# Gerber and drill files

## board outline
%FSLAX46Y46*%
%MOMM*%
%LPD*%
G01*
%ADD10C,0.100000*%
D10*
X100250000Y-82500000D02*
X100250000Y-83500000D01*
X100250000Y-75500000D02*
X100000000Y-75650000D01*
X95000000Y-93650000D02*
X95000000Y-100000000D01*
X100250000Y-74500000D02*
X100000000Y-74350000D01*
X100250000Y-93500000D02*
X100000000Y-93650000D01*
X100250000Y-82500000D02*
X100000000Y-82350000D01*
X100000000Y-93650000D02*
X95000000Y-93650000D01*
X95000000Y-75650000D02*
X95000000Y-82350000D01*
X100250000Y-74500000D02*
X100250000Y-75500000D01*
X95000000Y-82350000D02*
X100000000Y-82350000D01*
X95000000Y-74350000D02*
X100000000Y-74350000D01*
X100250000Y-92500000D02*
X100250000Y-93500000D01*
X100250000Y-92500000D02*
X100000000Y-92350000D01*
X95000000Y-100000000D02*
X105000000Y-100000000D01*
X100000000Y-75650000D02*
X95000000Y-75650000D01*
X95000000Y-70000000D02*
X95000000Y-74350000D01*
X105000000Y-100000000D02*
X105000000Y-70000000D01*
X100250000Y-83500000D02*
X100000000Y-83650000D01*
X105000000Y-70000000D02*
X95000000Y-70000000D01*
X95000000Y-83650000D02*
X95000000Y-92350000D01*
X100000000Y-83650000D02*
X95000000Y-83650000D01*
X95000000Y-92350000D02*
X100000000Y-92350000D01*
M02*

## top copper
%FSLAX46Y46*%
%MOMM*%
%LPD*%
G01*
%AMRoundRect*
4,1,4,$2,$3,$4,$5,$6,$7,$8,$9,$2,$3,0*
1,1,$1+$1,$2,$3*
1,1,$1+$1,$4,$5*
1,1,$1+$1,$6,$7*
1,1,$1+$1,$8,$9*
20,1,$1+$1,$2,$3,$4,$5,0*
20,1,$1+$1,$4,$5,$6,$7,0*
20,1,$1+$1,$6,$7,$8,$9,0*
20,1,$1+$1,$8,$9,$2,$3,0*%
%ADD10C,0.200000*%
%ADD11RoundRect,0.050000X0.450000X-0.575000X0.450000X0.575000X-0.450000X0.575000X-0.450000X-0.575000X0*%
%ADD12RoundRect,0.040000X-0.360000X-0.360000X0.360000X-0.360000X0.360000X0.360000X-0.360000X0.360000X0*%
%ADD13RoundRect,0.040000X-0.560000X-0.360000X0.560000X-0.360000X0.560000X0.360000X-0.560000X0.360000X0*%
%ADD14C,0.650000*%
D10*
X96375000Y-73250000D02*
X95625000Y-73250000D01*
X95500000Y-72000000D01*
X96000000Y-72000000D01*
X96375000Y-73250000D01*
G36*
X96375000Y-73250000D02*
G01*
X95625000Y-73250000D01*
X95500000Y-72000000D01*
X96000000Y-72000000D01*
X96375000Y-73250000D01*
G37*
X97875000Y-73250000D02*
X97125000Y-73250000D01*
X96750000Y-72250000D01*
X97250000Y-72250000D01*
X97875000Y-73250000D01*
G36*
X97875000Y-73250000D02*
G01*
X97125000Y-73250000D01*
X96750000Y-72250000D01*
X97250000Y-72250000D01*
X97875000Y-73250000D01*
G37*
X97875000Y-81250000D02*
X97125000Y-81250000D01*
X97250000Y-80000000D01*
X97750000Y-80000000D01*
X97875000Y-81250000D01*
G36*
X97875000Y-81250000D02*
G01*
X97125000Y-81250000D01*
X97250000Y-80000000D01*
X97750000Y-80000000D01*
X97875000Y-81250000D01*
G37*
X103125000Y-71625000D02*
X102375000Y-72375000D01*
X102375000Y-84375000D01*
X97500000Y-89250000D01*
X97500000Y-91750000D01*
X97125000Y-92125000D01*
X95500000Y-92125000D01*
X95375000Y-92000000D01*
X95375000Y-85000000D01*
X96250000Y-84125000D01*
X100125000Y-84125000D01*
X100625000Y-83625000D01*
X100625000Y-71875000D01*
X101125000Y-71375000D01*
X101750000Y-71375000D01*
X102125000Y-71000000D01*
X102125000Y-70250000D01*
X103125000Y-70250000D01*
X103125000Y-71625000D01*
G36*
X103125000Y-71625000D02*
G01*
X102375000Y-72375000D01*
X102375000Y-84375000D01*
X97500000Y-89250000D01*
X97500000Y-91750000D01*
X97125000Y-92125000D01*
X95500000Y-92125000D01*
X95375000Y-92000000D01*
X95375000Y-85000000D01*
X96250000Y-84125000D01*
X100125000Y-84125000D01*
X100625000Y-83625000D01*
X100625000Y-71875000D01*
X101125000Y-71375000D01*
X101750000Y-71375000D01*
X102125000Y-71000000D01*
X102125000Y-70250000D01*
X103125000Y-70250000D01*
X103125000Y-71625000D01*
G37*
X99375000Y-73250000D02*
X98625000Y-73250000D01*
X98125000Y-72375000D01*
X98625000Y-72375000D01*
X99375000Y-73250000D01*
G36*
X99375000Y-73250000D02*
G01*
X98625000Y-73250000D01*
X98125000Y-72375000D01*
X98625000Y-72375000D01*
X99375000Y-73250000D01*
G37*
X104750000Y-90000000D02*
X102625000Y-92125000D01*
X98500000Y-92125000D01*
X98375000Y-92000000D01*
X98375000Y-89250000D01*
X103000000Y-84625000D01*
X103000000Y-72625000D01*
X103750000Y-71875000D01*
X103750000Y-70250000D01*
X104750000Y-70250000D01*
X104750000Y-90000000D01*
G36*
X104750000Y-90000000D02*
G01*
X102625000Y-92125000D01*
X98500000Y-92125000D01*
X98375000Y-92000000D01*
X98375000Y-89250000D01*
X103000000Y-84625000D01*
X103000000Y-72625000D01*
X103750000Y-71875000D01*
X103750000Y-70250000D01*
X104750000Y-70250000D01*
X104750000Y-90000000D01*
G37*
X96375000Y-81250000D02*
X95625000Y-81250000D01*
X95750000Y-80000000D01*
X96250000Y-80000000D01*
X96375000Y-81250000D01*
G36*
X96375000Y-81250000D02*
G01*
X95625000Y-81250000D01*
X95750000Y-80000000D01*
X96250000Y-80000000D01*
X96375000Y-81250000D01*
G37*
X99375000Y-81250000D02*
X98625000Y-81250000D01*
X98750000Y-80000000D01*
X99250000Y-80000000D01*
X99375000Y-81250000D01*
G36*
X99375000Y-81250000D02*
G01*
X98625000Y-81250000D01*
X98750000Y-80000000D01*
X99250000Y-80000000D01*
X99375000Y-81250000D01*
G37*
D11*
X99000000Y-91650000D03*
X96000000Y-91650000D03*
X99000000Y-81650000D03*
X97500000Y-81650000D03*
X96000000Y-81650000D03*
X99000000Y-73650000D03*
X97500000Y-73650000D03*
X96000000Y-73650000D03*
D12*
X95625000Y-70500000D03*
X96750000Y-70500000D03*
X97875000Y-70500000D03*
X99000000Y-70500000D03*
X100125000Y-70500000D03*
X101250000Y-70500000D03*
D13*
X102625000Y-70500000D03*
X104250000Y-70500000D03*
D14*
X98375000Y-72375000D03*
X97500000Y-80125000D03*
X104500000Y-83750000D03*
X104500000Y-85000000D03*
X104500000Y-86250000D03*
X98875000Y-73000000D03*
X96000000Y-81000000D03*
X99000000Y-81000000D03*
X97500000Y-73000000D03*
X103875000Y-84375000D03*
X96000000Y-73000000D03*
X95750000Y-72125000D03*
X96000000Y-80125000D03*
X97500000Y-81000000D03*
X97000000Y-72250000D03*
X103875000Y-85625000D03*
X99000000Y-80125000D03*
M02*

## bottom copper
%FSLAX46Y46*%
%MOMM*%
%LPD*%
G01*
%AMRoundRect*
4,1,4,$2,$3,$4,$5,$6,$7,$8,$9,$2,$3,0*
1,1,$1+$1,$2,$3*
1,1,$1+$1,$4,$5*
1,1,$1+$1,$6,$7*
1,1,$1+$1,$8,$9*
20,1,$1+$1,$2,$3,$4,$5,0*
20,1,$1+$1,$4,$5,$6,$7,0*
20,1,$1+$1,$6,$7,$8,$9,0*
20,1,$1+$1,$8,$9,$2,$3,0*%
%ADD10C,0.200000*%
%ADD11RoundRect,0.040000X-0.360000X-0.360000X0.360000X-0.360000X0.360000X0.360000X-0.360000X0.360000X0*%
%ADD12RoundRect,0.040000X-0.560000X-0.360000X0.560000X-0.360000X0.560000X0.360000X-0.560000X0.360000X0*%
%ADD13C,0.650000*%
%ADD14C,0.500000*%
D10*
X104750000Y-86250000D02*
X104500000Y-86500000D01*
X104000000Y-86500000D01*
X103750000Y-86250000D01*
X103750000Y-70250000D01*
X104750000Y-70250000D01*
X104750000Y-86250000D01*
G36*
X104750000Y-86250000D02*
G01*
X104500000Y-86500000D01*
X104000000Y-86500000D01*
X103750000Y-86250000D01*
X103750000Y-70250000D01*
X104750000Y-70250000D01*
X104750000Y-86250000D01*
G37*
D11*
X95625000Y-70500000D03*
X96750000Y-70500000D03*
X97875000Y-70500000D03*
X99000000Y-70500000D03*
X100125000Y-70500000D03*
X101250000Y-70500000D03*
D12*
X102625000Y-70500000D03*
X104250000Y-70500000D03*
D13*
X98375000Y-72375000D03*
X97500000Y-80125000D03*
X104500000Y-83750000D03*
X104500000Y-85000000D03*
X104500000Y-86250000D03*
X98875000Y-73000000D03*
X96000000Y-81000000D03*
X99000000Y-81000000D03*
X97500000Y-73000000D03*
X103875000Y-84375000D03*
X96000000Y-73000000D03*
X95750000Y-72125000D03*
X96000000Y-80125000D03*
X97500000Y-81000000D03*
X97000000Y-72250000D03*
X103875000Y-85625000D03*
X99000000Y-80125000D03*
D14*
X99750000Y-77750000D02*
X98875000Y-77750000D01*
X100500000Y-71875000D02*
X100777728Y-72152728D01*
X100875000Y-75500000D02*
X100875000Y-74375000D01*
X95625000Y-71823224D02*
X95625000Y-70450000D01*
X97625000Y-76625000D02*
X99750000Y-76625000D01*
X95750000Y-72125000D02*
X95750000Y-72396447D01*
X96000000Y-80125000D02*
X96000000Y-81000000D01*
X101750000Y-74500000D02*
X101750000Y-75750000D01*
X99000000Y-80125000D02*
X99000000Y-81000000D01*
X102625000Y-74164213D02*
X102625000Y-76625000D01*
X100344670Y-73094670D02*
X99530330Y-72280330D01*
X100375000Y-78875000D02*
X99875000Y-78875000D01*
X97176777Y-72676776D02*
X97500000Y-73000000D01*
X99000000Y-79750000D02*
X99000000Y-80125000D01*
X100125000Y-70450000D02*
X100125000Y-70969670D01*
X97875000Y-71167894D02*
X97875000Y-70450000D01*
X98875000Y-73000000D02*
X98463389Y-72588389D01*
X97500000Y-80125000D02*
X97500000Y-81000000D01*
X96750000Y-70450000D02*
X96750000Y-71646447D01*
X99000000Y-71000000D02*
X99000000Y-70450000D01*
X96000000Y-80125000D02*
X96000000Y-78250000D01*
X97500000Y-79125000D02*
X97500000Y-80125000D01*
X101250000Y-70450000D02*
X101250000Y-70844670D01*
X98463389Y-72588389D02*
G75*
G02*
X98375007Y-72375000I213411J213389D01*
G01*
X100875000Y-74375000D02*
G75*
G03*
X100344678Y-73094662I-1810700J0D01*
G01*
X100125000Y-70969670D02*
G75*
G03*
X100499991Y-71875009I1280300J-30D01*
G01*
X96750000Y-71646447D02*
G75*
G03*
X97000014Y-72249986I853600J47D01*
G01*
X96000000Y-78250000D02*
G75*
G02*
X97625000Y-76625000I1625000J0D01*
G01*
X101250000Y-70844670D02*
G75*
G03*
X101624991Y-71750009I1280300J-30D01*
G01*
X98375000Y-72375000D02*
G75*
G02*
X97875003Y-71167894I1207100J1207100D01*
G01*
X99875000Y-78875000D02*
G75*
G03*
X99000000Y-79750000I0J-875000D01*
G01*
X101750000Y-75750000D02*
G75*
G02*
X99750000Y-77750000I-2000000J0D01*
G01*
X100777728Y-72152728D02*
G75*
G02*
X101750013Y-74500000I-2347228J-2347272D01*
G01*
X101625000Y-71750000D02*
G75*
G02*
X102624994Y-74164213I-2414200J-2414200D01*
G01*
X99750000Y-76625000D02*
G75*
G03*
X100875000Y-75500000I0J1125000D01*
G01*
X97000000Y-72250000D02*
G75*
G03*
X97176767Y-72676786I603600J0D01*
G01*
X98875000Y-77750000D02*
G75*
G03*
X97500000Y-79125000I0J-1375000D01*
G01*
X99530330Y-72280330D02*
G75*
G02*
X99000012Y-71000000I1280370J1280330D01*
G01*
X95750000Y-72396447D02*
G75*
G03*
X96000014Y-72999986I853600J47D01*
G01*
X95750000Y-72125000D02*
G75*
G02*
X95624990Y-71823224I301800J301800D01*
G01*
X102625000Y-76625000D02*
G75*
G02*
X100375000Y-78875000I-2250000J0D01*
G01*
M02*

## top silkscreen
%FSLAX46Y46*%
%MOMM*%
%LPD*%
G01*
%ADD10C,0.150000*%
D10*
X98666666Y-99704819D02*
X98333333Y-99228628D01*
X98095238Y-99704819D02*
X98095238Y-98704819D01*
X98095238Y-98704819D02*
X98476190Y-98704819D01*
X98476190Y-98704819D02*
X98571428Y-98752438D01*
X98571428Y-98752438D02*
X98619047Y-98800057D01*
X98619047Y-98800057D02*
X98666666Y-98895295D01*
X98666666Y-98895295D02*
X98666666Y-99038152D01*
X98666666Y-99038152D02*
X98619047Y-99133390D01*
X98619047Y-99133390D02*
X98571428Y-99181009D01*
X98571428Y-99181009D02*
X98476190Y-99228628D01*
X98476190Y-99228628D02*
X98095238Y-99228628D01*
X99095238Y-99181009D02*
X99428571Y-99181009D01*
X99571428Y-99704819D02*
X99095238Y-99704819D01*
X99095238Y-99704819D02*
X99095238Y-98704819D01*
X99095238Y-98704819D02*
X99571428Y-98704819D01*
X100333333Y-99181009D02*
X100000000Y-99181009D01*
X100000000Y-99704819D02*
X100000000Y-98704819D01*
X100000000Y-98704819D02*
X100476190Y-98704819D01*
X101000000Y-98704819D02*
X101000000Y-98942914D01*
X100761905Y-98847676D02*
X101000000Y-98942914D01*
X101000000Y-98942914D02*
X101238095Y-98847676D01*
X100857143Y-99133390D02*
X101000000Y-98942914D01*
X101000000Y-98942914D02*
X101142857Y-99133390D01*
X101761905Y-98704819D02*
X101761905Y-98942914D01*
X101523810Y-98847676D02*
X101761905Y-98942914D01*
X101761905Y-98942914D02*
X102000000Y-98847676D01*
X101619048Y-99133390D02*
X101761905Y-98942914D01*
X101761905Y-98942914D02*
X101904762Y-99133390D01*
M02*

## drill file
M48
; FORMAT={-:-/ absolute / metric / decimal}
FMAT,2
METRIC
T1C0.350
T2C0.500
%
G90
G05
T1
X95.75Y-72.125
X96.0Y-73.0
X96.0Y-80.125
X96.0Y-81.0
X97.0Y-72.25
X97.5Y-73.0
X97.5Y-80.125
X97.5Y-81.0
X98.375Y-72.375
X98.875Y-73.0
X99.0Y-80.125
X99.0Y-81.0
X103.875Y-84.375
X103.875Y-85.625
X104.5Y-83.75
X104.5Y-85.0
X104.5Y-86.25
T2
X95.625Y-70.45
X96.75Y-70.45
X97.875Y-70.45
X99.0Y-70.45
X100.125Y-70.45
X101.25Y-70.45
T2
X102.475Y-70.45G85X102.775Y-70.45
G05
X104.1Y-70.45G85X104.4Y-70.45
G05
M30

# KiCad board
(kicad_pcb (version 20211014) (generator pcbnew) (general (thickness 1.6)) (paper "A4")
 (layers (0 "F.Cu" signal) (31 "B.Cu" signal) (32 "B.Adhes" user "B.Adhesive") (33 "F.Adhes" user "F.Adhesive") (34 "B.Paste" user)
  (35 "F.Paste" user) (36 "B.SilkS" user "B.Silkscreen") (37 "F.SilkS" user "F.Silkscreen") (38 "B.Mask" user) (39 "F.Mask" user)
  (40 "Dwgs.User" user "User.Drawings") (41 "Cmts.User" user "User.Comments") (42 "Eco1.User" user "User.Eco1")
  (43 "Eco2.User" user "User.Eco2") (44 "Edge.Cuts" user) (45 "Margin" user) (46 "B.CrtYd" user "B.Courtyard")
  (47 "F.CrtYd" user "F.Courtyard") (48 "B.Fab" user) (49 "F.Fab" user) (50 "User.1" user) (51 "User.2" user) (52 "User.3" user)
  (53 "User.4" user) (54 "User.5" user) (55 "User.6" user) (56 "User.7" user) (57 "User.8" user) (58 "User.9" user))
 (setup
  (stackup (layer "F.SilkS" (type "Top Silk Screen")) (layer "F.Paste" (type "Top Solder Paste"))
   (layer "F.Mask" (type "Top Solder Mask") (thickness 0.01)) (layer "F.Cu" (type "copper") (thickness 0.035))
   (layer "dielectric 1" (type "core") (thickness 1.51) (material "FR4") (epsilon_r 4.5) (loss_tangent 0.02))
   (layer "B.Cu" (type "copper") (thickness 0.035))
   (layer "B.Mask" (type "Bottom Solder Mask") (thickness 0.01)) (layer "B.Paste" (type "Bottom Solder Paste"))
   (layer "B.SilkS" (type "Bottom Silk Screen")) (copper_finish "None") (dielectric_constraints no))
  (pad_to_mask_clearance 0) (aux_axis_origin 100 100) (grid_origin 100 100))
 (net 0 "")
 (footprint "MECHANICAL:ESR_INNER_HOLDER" (layer "F.Cu") (at 100 100)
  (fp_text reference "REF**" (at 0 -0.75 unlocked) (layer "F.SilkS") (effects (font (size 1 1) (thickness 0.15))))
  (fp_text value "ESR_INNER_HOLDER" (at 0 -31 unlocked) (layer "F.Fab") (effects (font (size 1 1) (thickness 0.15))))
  (fp_line (start 0.25 -17.5) (end 0.25 -16.5) (layer "Edge.Cuts") (width 0.1))
  (fp_line (start 0.25 -24.5) (end 0 -24.35) (layer "Edge.Cuts") (width 0.1))
  (fp_line (start -5 -6.35) (end -5 0) (layer "Edge.Cuts") (width 0.1))
  (fp_line (start 0.25 -25.5) (end 0 -25.65) (layer "Edge.Cuts") (width 0.1))
  (fp_line (start 0.25 -6.5) (end 0 -6.35) (layer "Edge.Cuts") (width 0.1))
  (fp_line (start 0.25 -17.5) (end 0 -17.65) (layer "Edge.Cuts") (width 0.1))
  (fp_line (start 0 -6.35) (end -5 -6.35) (layer "Edge.Cuts") (width 0.1))
  (fp_line (start -5 -24.35) (end -5 -17.65) (layer "Edge.Cuts") (width 0.1))
  (fp_line (start 0.25 -25.5) (end 0.25 -24.5) (layer "Edge.Cuts") (width 0.1))
  (fp_line (start -5 -17.65) (end 0 -17.65) (layer "Edge.Cuts") (width 0.1))
  (fp_line (start -5 -25.65) (end 0 -25.65) (layer "Edge.Cuts") (width 0.1))
  (fp_line (start 0.25 -7.5) (end 0.25 -6.5) (layer "Edge.Cuts") (width 0.1))
  (fp_line (start 0.25 -7.5) (end 0 -7.65) (layer "Edge.Cuts") (width 0.1))
  (fp_line (start -5 0) (end 5 0) (layer "Edge.Cuts") (width 0.1))
  (fp_line (start 0 -24.35) (end -5 -24.35) (layer "Edge.Cuts") (width 0.1))
  (fp_line (start -5 -30) (end -5 -25.65) (layer "Edge.Cuts") (width 0.1))
  (fp_line (start 5 0) (end 5 -30) (layer "Edge.Cuts") (width 0.1))
  (fp_line (start 0.25 -16.5) (end 0 -16.35) (layer "Edge.Cuts") (width 0.1))
  (fp_line (start 5 -30) (end -5 -30) (layer "Edge.Cuts") (width 0.1))
  (fp_line (start -5 -16.35) (end -5 -7.65) (layer "Edge.Cuts") (width 0.1))
  (fp_line (start 0 -16.35) (end -5 -16.35) (layer "Edge.Cuts") (width 0.1))
  (fp_line (start -5 -7.65) (end 0 -7.65) (layer "Edge.Cuts") (width 0.1))
  (pad "1" smd roundrect (at -1 -8.35 90) (size 1.25 1) (layers "F.Cu" "F.Paste" "F.Mask") (roundrect_rratio 0.05) (solder_mask_margin 0.05)
   (solder_paste_margin_ratio -0.1))
  (pad "3" smd roundrect (at -4 -8.35 90) (size 1.25 1) (layers "F.Cu" "F.Paste" "F.Mask") (roundrect_rratio 0.05) (solder_mask_margin 0.05)
   (solder_paste_margin_ratio -0.1))
  (pad "4" smd roundrect (at -1 -18.35 90) (size 1.25 1) (layers "F.Cu" "F.Paste" "F.Mask") (roundrect_rratio 0.05)
   (solder_mask_margin 0.05) (solder_paste_margin_ratio -0.1))
  (pad "5" smd roundrect (at -2.5 -18.35 90) (size 1.25 1) (layers "F.Cu" "F.Paste" "F.Mask") (roundrect_rratio 0.05)
   (solder_mask_margin 0.05) (solder_paste_margin_ratio -0.1))
  (pad "6" smd roundrect (at -4 -18.35 90) (size 1.25 1) (layers "F.Cu" "F.Paste" "F.Mask") (roundrect_rratio 0.05)
   (solder_mask_margin 0.05) (solder_paste_margin_ratio -0.1))
  (pad "7" smd roundrect (at -1 -26.35 90) (size 1.25 1) (layers "F.Cu" "F.Paste" "F.Mask") (roundrect_rratio 0.05)
   (solder_mask_margin 0.05) (solder_paste_margin_ratio -0.1))
  (pad "8" smd roundrect (at -2.5 -26.35 90) (size 1.25 1) (layers "F.Cu" "F.Paste" "F.Mask") (roundrect_rratio 0.05)
   (solder_mask_margin 0.05) (solder_paste_margin_ratio -0.1))
  (pad "9" smd roundrect (at -4 -26.35 90) (size 1.25 1) (layers "F.Cu" "F.Paste" "F.Mask") (roundrect_rratio 0.05)
   (solder_mask_margin 0.05) (solder_paste_margin_ratio -0.1))
  (pad "A" thru_hole roundrect (at -4.375 -29.55) (size 0.8 0.8) (drill 0.5 (offset 0 0.05)) (layers *.Cu *.Mask) (roundrect_rratio 0.05)
   (solder_mask_margin 0.05) (solder_paste_margin_ratio -0.1))
  (pad "B" thru_hole roundrect (at -3.25 -29.55) (size 0.8 0.8) (drill 0.5 (offset 0 0.05)) (layers *.Cu *.Mask) (roundrect_rratio 0.05)
   (solder_mask_margin 0.05) (solder_paste_margin_ratio -0.1))
  (pad "C" thru_hole roundrect (at -2.125 -29.55) (size 0.8 0.8) (drill 0.5 (offset 0 0.05)) (layers *.Cu *.Mask) (roundrect_rratio 0.05)
   (solder_mask_margin 0.05) (solder_paste_margin_ratio -0.1))
  (pad "D" thru_hole roundrect (at -1 -29.55) (size 0.8 0.8) (drill 0.5 (offset 0 0.05)) (layers *.Cu *.Mask) (roundrect_rratio 0.05)
   (solder_mask_margin 0.05) (solder_paste_margin_ratio -0.1))
  (pad "E" thru_hole roundrect (at 0.125 -29.55) (size 0.8 0.8) (drill 0.5 (offset 0 0.05)) (layers *.Cu *.Mask) (roundrect_rratio 0.05)
   (solder_mask_margin 0.05) (solder_paste_margin_ratio -0.1))
  (pad "F" thru_hole roundrect (at 1.25 -29.55) (size 0.8 0.8) (drill 0.5 (offset 0 0.05)) (layers *.Cu *.Mask) (roundrect_rratio 0.05)
   (solder_mask_margin 0.05) (solder_paste_margin_ratio -0.1))
  (pad "G" thru_hole roundrect (at 2.625 -29.55) (size 1.2 0.8) (drill oval 0.8 0.5 (offset 0 0.05)) (layers *.Cu *.Mask)
   (roundrect_rratio 0.05) (solder_mask_margin 0.05) (solder_paste_margin_ratio -0.1))
  (pad "H" thru_hole roundrect (at 4.25 -29.55) (size 1.2 0.8) (drill oval 0.8 0.5 (offset 0 0.05)) (layers *.Cu *.Mask)
   (roundrect_rratio 0.05) (solder_mask_margin 0.05) (solder_paste_margin_ratio -0.1)))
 (gr_poly (pts (xy 96.375 73.25) (xy 95.625 73.25) (xy 95.5 72) (xy 96 72)) (layer "F.Cu") (width 0.2) (fill solid))
 (gr_poly (pts (xy 97.875 73.25) (xy 97.125 73.25) (xy 96.75 72.25) (xy 97.25 72.25)) (layer "F.Cu") (width 0.2) (fill solid))
 (gr_poly (pts (xy 97.875 81.25) (xy 97.125 81.25) (xy 97.25 80) (xy 97.75 80)) (layer "F.Cu") (width 0.2) (fill solid))
 (gr_poly
  (pts (xy 103.125 71.625) (xy 102.375 72.375) (xy 102.375 84.375) (xy 97.5 89.25) (xy 97.5 91.75) (xy 97.125 92.125) (xy 95.5 92.125)
   (xy 95.375 92) (xy 95.375 85) (xy 96.25 84.125) (xy 100.125 84.125) (xy 100.625 83.625) (xy 100.625 71.875) (xy 101.125 71.375)
   (xy 101.75 71.375) (xy 102.125 71) (xy 102.125 70.25) (xy 103.125 70.25))
  (layer "F.Cu") (width 0.2) (fill solid))
 (gr_poly (pts (xy 99.375 73.25) (xy 98.625 73.25) (xy 98.125 72.375) (xy 98.625 72.375)) (layer "F.Cu") (width 0.2) (fill solid))
 (gr_poly
  (pts (xy 104.75 90) (xy 102.625 92.125) (xy 98.5 92.125) (xy 98.375 92) (xy 98.375 89.25) (xy 103 84.625) (xy 103 72.625)
   (xy 103.75 71.875) (xy 103.75 70.25) (xy 104.75 70.25))
  (layer "F.Cu") (width 0.2) (fill solid))
 (gr_poly (pts (xy 96.375 81.25) (xy 95.625 81.25) (xy 95.75 80) (xy 96.25 80)) (layer "F.Cu") (width 0.2) (fill solid))
 (gr_poly (pts (xy 99.375 81.25) (xy 98.625 81.25) (xy 98.75 80) (xy 99.25 80)) (layer "F.Cu") (width 0.2) (fill solid))
 (gr_poly
  (pts (xy 104.75 86.25) (xy 104.5 86.5) (xy 104 86.5) (xy 103.75 86.25) (xy 103.75 70.25) (xy 104.75 70.25)) (layer "B.Cu") (width 0.2)
  (fill solid))
 (via (at 98.375 72.375) (size 0.65) (drill 0.35) (layers "F.Cu" "B.Cu") (free) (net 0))
 (via (at 97.5 80.125) (size 0.65) (drill 0.35) (layers "F.Cu" "B.Cu") (free) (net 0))
 (via (at 104.5 83.75) (size 0.65) (drill 0.35) (layers "F.Cu" "B.Cu") (free) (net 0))
 (via (at 104.5 85) (size 0.65) (drill 0.35) (layers "F.Cu" "B.Cu") (free) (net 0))
 (via (at 104.5 86.25) (size 0.65) (drill 0.35) (layers "F.Cu" "B.Cu") (free) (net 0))
 (via (at 98.875 73) (size 0.65) (drill 0.35) (layers "F.Cu" "B.Cu") (free) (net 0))
 (via (at 96 81) (size 0.65) (drill 0.35) (layers "F.Cu" "B.Cu") (free) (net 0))
 (via (at 99 81) (size 0.65) (drill 0.35) (layers "F.Cu" "B.Cu") (free) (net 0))
 (via (at 97.5 73) (size 0.65) (drill 0.35) (layers "F.Cu" "B.Cu") (free) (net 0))
 (via (at 103.875 84.375) (size 0.65) (drill 0.35) (layers "F.Cu" "B.Cu") (free) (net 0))
 (via (at 96 73) (size 0.65) (drill 0.35) (layers "F.Cu" "B.Cu") (free) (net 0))
 (via (at 95.75 72.125) (size 0.65) (drill 0.35) (layers "F.Cu" "B.Cu") (free) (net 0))
 (via (at 96 80.125) (size 0.65) (drill 0.35) (layers "F.Cu" "B.Cu") (free) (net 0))
 (via (at 97.5 81) (size 0.65) (drill 0.35) (layers "F.Cu" "B.Cu") (free) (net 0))
 (via (at 97 72.25) (size 0.65) (drill 0.35) (layers "F.Cu" "B.Cu") (free) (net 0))
 (via (at 103.875 85.625) (size 0.65) (drill 0.35) (layers "F.Cu" "B.Cu") (free) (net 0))
 (via (at 99 80.125) (size 0.65) (drill 0.35) (layers "F.Cu" "B.Cu") (free) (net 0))
 (segment (start 99.75 77.75) (end 98.875 77.75) (width 0.5) (layer "B.Cu") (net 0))
 (segment (start 100.5 71.875) (end 100.777728 72.152728) (width 0.5) (layer "B.Cu") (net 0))
 (segment (start 100.875 75.5) (end 100.875 74.375) (width 0.5) (layer "B.Cu") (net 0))
 (segment (start 95.625 71.823224) (end 95.625 70.45) (width 0.5) (layer "B.Cu") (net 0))
 (segment (start 97.625 76.625) (end 99.75 76.625) (width 0.5) (layer "B.Cu") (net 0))
 (segment (start 95.75 72.125) (end 95.75 72.396447) (width 0.5) (layer "B.Cu") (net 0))
 (segment (start 96 80.125) (end 96 81) (width 0.5) (layer "B.Cu") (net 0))
 (segment (start 101.75 74.5) (end 101.75 75.75) (width 0.5) (layer "B.Cu") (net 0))
 (segment (start 99 80.125) (end 99 81) (width 0.5) (layer "B.Cu") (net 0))
 (segment (start 102.625 74.164213) (end 102.625 76.625) (width 0.5) (layer "B.Cu") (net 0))
 (segment (start 100.34467 73.09467) (end 99.53033 72.28033) (width 0.5) (layer "B.Cu") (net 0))
 (segment (start 100.375 78.875) (end 99.875 78.875) (width 0.5) (layer "B.Cu") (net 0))
 (segment (start 97.176777 72.676776) (end 97.5 73) (width 0.5) (layer "B.Cu") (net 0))
 (segment (start 99 79.75) (end 99 80.125) (width 0.5) (layer "B.Cu") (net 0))
 (segment (start 100.125 70.45) (end 100.125 70.96967) (width 0.5) (layer "B.Cu") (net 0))
 (segment (start 97.875 71.167894) (end 97.875 70.45) (width 0.5) (layer "B.Cu") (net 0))
 (segment (start 98.875 73) (end 98.463389 72.588389) (width 0.5) (layer "B.Cu") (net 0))
 (segment (start 97.5 80.125) (end 97.5 81) (width 0.5) (layer "B.Cu") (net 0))
 (segment (start 96.75 70.45) (end 96.75 71.646447) (width 0.5) (layer "B.Cu") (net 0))
 (segment (start 99 71) (end 99 70.45) (width 0.5) (layer "B.Cu") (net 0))
 (segment (start 96 80.125) (end 96 78.25) (width 0.5) (layer "B.Cu") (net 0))
 (segment (start 97.5 79.125) (end 97.5 80.125) (width 0.5) (layer "B.Cu") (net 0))
 (segment (start 101.25 70.45) (end 101.25 70.84467) (width 0.5) (layer "B.Cu") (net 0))
 (arc (start 98.463389 72.588389) (mid 98.397971 72.490486) (end 98.375 72.375) (width 0.5) (layer "B.Cu") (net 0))
 (arc (start 100.875 74.375) (mid 100.737172 73.68209) (end 100.34467 73.09467) (width 0.5) (layer "B.Cu") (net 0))
 (arc (start 100.125 70.96967) (mid 100.22246 71.459631) (end 100.5 71.875) (width 0.5) (layer "B.Cu") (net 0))
 (arc (start 96.75 71.646447) (mid 96.814973 71.973087) (end 97 72.25) (width 0.5) (layer "B.Cu") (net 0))
 (arc (start 96 78.25) (mid 96.475951 77.100951) (end 97.625 76.625) (width 0.5) (layer "B.Cu") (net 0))
 (arc (start 101.25 70.84467) (mid 101.34746 71.334631) (end 101.625 71.75) (width 0.5) (layer "B.Cu") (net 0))
 (arc (start 98.375 72.375) (mid 98.004946 71.821175) (end 97.875 71.167894) (width 0.5) (layer "B.Cu") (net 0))
 (arc (start 99.875 78.875) (mid 99.256282 79.131282) (end 99 79.75) (width 0.5) (layer "B.Cu") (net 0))
 (arc (start 101.75 75.75) (mid 101.164214 77.164214) (end 99.75 77.75) (width 0.5) (layer "B.Cu") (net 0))
 (arc (start 100.777728 72.152728) (mid 101.497315 73.229666) (end 101.75 74.5) (width 0.5) (layer "B.Cu") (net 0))
 (arc (start 101.625 71.75) (mid 102.365108 72.85765) (end 102.625 74.164213) (width 0.5) (layer "B.Cu") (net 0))
 (arc (start 99.75 76.625) (mid 100.545495 76.295495) (end 100.875 75.5) (width 0.5) (layer "B.Cu") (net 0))
 (arc (start 97 72.25) (mid 97.045943 72.48097) (end 97.176777 72.676776) (width 0.5) (layer "B.Cu") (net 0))
 (arc (start 98.875 77.75) (mid 97.902728 78.152728) (end 97.5 79.125) (width 0.5) (layer "B.Cu") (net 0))
 (arc (start 99.53033 72.28033) (mid 99.137828 71.69291) (end 99 71) (width 0.5) (layer "B.Cu") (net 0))
 (arc (start 95.75 72.396447) (mid 95.814973 72.723087) (end 96 73) (width 0.5) (layer "B.Cu") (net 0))
 (arc (start 95.75 72.125) (mid 95.657486 71.986544) (end 95.625 71.823224) (width 0.5) (layer "B.Cu") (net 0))
 (arc (start 102.625 76.625) (mid 101.96599 78.21599) (end 100.375 78.875) (width 0.5) (layer "B.Cu") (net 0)))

